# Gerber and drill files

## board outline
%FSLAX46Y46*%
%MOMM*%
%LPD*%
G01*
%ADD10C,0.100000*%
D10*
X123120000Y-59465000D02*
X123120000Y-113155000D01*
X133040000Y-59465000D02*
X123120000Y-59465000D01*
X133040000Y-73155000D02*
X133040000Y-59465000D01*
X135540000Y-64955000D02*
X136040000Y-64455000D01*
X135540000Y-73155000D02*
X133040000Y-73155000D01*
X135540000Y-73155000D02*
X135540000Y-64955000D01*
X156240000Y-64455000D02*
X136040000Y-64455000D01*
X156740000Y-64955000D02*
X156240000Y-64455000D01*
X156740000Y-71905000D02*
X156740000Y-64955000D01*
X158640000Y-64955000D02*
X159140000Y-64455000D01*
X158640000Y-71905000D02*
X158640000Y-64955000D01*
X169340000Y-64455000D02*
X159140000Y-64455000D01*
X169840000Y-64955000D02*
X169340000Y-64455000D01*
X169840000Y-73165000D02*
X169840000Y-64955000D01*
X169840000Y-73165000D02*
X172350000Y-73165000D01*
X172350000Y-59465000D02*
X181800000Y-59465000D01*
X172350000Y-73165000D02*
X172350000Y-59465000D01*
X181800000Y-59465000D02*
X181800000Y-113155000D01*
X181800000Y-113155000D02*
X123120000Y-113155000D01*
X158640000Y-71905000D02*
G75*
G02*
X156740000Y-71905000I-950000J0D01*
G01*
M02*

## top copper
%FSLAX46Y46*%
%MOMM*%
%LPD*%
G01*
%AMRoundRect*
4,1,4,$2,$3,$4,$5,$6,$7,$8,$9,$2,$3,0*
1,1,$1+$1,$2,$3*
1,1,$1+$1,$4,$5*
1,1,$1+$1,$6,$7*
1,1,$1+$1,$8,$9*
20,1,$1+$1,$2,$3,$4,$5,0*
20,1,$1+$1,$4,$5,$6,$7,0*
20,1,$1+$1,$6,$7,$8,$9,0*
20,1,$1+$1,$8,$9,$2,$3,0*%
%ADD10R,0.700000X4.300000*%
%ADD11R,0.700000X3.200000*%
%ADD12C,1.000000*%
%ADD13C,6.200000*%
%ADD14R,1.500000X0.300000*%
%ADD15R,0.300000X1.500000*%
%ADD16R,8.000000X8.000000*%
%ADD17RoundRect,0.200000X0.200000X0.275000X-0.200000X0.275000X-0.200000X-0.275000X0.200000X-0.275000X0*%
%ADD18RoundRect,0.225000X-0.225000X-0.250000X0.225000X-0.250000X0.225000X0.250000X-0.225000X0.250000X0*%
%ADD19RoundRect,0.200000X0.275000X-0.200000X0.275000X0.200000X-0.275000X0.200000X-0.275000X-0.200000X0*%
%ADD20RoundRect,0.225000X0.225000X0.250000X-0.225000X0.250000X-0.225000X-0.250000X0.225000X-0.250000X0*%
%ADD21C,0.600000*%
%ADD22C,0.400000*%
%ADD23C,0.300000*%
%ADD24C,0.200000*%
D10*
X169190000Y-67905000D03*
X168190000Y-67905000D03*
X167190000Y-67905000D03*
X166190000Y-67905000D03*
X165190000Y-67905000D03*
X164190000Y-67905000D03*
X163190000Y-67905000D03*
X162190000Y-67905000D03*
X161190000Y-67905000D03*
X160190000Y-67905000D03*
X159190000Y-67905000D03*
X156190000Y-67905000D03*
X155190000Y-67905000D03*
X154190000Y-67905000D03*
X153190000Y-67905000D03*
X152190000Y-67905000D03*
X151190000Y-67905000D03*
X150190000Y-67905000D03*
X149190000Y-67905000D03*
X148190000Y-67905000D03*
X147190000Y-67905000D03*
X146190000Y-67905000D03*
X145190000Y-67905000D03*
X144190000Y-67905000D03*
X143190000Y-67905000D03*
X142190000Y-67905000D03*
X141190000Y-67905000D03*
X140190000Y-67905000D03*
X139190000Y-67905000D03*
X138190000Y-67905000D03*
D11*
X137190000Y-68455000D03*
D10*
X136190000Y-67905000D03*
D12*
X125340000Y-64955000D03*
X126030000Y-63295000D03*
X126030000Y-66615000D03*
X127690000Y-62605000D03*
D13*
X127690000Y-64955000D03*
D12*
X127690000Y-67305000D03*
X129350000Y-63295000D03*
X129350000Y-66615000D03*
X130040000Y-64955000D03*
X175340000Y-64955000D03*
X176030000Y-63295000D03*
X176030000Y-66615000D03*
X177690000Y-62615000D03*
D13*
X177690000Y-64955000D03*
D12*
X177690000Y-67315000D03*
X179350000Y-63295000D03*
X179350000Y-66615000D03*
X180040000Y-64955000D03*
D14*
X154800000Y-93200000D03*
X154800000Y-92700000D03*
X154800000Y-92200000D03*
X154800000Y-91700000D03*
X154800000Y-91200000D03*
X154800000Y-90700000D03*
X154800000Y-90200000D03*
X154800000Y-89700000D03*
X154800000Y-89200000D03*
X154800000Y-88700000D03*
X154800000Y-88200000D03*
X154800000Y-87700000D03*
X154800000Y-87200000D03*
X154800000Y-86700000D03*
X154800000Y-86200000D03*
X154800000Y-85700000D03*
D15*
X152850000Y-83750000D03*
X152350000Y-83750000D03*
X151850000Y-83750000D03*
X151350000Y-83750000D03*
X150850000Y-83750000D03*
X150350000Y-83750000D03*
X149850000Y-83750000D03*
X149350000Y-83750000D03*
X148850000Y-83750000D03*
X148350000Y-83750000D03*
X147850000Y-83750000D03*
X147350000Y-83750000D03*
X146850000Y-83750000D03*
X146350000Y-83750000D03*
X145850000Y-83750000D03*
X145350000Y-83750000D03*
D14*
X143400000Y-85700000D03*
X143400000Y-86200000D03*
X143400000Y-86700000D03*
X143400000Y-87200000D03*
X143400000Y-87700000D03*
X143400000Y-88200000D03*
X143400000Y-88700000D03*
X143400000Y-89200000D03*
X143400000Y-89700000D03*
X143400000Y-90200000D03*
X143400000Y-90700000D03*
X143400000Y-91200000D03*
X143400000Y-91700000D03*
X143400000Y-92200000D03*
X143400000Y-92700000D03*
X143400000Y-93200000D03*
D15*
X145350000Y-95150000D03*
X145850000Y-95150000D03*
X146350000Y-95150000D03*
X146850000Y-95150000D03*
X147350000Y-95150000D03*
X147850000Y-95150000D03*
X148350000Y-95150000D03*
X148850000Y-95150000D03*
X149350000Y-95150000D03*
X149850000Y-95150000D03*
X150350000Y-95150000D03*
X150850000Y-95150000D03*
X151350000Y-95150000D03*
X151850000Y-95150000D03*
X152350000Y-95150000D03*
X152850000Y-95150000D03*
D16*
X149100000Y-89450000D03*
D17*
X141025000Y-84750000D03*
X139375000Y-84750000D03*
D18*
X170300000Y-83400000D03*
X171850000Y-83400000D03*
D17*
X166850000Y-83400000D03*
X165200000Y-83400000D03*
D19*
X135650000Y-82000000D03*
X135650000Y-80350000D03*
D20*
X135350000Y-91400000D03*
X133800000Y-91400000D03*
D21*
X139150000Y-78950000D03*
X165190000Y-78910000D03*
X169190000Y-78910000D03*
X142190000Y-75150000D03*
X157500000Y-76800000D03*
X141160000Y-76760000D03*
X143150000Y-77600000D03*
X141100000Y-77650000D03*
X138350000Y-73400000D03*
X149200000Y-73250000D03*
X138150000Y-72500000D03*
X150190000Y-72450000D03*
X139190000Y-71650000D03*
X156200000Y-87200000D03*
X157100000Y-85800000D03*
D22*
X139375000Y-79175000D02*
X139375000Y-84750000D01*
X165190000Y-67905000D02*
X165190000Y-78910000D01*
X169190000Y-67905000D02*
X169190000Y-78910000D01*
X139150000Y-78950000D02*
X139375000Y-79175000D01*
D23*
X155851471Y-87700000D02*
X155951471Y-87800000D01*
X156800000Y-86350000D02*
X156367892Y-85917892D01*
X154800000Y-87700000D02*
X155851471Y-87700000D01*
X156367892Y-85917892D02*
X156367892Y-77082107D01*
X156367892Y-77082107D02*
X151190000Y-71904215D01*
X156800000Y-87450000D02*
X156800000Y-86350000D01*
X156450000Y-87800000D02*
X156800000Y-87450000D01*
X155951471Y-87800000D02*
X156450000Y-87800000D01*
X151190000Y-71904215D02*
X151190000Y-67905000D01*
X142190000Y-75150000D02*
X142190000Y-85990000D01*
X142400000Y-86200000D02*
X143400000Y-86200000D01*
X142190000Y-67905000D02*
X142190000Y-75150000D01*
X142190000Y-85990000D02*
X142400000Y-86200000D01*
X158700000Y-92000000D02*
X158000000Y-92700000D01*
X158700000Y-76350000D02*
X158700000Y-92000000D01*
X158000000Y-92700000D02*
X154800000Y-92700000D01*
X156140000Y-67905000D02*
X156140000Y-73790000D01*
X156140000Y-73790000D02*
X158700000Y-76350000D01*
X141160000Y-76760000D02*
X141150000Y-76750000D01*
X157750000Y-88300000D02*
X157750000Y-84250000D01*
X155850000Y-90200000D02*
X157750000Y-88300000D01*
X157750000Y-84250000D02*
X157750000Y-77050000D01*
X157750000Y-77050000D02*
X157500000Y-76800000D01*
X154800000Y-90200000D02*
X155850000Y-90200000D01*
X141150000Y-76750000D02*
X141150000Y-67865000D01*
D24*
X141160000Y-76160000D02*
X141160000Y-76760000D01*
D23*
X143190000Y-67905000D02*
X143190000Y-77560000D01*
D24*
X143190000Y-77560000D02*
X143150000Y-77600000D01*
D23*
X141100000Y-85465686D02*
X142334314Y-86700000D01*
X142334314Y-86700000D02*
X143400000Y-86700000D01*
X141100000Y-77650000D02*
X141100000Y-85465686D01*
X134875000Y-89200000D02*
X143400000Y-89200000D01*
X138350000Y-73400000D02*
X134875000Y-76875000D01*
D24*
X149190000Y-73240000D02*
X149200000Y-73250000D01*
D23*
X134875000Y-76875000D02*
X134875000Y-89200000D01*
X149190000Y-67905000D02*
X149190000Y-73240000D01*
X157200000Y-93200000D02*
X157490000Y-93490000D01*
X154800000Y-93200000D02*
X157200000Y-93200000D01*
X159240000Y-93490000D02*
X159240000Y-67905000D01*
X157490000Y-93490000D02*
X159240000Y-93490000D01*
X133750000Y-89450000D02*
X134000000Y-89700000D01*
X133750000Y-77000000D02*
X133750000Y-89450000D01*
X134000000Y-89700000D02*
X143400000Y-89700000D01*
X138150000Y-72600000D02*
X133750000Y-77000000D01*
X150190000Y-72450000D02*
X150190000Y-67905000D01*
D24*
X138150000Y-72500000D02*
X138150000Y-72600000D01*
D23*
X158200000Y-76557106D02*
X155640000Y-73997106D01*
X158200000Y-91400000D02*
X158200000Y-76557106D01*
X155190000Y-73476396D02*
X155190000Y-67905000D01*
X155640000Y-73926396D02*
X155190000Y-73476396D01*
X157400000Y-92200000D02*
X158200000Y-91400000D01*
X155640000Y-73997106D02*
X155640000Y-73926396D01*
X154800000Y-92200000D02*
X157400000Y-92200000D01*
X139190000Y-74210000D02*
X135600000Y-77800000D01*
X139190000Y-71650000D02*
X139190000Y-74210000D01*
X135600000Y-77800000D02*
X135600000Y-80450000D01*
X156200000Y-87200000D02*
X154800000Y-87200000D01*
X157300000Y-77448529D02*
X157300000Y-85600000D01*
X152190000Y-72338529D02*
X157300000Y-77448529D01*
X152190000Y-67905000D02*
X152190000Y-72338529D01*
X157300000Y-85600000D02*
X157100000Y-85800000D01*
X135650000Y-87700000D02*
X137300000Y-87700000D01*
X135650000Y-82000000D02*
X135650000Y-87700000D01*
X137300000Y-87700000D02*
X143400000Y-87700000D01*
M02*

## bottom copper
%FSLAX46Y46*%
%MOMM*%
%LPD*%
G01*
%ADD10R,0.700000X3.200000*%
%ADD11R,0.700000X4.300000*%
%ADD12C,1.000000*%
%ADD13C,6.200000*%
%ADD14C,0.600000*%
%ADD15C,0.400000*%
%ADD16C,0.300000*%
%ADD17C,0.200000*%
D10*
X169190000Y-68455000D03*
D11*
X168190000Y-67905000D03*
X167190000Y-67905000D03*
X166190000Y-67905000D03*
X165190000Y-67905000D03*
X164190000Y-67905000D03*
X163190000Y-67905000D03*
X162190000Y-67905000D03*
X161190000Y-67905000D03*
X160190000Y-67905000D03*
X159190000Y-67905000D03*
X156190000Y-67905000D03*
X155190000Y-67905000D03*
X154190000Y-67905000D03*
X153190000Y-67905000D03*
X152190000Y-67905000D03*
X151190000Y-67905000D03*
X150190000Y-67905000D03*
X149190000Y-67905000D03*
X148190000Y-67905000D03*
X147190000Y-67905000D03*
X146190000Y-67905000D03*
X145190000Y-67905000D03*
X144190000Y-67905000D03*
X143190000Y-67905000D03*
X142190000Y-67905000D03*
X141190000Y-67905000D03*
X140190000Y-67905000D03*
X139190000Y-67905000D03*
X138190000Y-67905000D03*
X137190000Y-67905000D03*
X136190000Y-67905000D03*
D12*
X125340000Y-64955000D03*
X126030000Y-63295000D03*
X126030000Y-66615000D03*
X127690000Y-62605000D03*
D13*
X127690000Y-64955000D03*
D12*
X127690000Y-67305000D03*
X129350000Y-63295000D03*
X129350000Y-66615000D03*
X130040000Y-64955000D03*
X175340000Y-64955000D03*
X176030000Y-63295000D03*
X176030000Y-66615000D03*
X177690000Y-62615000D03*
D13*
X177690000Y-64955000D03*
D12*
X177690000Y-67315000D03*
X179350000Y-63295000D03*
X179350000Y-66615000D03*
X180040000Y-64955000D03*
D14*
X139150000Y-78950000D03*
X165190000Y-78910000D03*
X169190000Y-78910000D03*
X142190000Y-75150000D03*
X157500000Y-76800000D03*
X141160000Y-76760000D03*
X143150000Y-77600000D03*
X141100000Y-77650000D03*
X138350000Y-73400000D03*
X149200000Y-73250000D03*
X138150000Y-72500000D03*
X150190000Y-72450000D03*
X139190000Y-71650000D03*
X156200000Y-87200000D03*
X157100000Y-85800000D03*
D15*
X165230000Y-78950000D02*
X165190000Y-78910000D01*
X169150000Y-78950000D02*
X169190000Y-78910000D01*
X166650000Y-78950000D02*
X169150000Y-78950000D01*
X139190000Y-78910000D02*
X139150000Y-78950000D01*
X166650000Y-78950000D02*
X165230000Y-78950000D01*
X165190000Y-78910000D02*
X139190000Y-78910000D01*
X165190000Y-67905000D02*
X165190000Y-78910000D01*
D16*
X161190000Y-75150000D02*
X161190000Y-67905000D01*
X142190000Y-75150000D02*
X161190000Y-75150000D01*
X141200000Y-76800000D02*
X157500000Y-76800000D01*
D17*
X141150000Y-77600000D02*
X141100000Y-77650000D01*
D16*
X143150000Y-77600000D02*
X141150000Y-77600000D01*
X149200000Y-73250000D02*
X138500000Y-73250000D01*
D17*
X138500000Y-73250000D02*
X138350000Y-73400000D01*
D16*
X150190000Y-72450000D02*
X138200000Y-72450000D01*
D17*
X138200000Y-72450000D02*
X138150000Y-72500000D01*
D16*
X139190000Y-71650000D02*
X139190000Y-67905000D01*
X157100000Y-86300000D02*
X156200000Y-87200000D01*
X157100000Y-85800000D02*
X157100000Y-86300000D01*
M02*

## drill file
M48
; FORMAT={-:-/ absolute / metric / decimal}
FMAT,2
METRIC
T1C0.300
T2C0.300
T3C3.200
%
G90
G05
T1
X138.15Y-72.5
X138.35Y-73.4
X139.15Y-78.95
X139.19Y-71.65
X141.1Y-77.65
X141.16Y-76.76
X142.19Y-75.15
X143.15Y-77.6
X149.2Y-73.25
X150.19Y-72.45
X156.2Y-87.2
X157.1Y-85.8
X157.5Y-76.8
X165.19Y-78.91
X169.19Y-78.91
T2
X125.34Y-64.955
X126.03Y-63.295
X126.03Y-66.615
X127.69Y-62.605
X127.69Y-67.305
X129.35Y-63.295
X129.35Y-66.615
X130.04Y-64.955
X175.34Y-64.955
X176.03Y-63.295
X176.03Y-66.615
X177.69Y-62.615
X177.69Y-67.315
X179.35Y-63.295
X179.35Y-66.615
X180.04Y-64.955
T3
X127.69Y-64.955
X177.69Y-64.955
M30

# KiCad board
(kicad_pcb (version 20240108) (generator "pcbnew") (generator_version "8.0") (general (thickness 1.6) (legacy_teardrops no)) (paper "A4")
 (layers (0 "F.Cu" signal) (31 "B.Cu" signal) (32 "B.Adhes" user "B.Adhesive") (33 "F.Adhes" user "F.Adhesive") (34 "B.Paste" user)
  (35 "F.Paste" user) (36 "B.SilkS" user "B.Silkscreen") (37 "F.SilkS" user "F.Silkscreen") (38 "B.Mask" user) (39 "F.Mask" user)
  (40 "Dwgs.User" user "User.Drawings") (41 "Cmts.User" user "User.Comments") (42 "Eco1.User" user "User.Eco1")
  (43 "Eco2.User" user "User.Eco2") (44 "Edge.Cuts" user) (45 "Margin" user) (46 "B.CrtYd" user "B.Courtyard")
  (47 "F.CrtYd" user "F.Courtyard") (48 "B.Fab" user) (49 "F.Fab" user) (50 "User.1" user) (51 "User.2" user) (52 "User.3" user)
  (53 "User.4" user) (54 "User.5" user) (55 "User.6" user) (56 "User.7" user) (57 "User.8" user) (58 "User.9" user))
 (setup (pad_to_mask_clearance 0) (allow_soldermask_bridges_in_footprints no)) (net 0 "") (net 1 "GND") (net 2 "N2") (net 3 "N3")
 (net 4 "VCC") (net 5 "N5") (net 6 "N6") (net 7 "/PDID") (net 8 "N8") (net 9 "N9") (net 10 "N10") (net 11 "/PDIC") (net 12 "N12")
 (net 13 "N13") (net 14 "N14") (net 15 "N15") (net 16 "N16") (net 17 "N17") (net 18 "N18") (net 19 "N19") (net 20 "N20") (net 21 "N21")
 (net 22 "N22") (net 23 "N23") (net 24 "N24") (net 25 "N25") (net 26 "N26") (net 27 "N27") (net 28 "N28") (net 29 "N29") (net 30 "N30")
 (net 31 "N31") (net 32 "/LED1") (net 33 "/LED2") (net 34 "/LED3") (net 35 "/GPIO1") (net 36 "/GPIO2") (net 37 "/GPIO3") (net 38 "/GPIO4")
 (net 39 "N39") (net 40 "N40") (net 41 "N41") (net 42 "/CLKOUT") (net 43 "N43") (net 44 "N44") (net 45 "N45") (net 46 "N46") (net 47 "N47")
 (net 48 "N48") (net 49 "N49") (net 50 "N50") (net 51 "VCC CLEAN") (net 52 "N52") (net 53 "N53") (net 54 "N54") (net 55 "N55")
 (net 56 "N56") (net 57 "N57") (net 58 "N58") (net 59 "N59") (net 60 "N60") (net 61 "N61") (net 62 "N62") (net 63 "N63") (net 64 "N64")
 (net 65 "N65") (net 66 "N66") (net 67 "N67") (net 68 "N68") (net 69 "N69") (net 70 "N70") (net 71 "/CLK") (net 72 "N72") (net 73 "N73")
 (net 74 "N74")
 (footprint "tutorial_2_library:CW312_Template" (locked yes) (layer "F.Cu") (at 127.69 64.955)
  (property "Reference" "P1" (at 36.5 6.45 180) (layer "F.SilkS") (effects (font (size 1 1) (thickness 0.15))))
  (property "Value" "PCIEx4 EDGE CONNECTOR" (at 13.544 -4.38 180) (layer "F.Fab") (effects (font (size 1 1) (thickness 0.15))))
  (fp_line (start -4.57 -5.49) (end -4.57 48.2) (stroke (width 0.1) (type default)) (layer "Edge.Cuts"))
  (fp_line (start 5.35 -5.49) (end -4.57 -5.49) (stroke (width 0.1) (type default)) (layer "Edge.Cuts"))
  (fp_line (start 5.35 8.2) (end 5.35 -5.49) (stroke (width 0.1) (type default)) (layer "Edge.Cuts"))
  (fp_line (start 7.85 0) (end 8.35 -0.5) (stroke (width 0.1) (type solid)) (layer "Edge.Cuts"))
  (fp_line (start 7.85 8.2) (end 5.35 8.2) (stroke (width 0.1) (type default)) (layer "Edge.Cuts"))
  (fp_line (start 7.85 8.2) (end 7.85 0) (stroke (width 0.1) (type solid)) (layer "Edge.Cuts"))
  (fp_line (start 28.55 -0.5) (end 8.35 -0.5) (stroke (width 0.1) (type solid)) (layer "Edge.Cuts"))
  (fp_line (start 29.05 0) (end 28.55 -0.5) (stroke (width 0.1) (type solid)) (layer "Edge.Cuts"))
  (fp_line (start 29.05 6.95) (end 29.05 0) (stroke (width 0.1) (type solid)) (layer "Edge.Cuts"))
  (fp_line (start 30.95 0) (end 31.45 -0.5) (stroke (width 0.1) (type solid)) (layer "Edge.Cuts"))
  (fp_line (start 30.95 6.95) (end 30.95 0) (stroke (width 0.1) (type solid)) (layer "Edge.Cuts"))
  (fp_line (start 41.65 -0.5) (end 31.45 -0.5) (stroke (width 0.1) (type solid)) (layer "Edge.Cuts"))
  (fp_line (start 42.15 0) (end 41.65 -0.5) (stroke (width 0.1) (type solid)) (layer "Edge.Cuts"))
  (fp_line (start 42.15 8.21) (end 42.15 0) (stroke (width 0.1) (type solid)) (layer "Edge.Cuts"))
  (fp_line (start 42.15 8.21) (end 44.66 8.21) (stroke (width 0.1) (type default)) (layer "Edge.Cuts"))
  (fp_line (start 44.66 -5.49) (end 54.11 -5.49) (stroke (width 0.1) (type default)) (layer "Edge.Cuts"))
  (fp_line (start 44.66 8.21) (end 44.66 -5.49) (stroke (width 0.1) (type default)) (layer "Edge.Cuts"))
  (fp_line (start 54.11 -5.49) (end 54.11 48.2) (stroke (width 0.1) (type default)) (layer "Edge.Cuts"))
  (fp_line (start 54.11 48.2) (end -4.57 48.2) (stroke (width 0.1) (type default)) (layer "Edge.Cuts"))
  (fp_arc (start 30.95 6.95) (mid 30 7.9) (end 29.05 6.95) (stroke (width 0.1) (type solid)) (layer "Edge.Cuts"))
  (pad "A1" connect rect (at 41.5 3.5 180) (size 0.7 3.2) (layers "B.Cu" "B.Mask") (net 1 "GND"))
  (pad "A2" connect rect (at 40.5 2.95 180) (size 0.7 4.3) (layers "B.Cu" "B.Mask") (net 1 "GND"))
  (pad "A3" connect rect (at 39.5 2.95 180) (size 0.7 4.3) (layers "B.Cu" "B.Mask") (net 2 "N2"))
  (pad "A4" connect rect (at 38.5 2.95 180) (size 0.7 4.3) (layers "B.Cu" "B.Mask") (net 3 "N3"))
  (pad "A5" connect rect (at 37.5 2.95 180) (size 0.7 4.3) (layers "B.Cu" "B.Mask") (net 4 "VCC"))
  (pad "A6" connect rect (at 36.5 2.95 180) (size 0.7 4.3) (layers "B.Cu" "B.Mask") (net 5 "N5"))
  (pad "A7" connect rect (at 35.5 2.95 180) (size 0.7 4.3) (layers "B.Cu" "B.Mask") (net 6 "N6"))
  (pad "A8" connect rect (at 34.5 2.95 180) (size 0.7 4.3) (layers "B.Cu" "B.Mask") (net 1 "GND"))
  (pad "A9" connect rect (at 33.5 2.95 180) (size 0.7 4.3) (layers "B.Cu" "B.Mask") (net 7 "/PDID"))
  (pad "A10" connect rect (at 32.5 2.95 180) (size 0.7 4.3) (layers "B.Cu" "B.Mask") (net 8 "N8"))
  (pad "A11" connect rect (at 31.5 2.95 180) (size 0.7 4.3) (layers "B.Cu" "B.Mask") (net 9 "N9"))
  (pad "A12" connect rect (at 28.5 2.95 180) (size 0.7 4.3) (layers "B.Cu" "B.Mask") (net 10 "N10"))
  (pad "A13" connect rect (at 27.5 2.95 180) (size 0.7 4.3) (layers "B.Cu" "B.Mask") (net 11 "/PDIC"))
  (pad "A14" connect rect (at 26.5 2.95 180) (size 0.7 4.3) (layers "B.Cu" "B.Mask") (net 1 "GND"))
  (pad "A15" connect rect (at 25.5 2.95 180) (size 0.7 4.3) (layers "B.Cu" "B.Mask") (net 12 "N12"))
  (pad "A16" connect rect (at 24.5 2.95 180) (size 0.7 4.3) (layers "B.Cu" "B.Mask") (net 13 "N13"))
  (pad "A17" connect rect (at 23.5 2.95 180) (size 0.7 4.3) (layers "B.Cu" "B.Mask") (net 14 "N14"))
  (pad "A18" connect rect (at 22.5 2.95 180) (size 0.7 4.3) (layers "B.Cu" "B.Mask") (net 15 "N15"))
  (pad "A19" connect rect (at 21.5 2.95 180) (size 0.7 4.3) (layers "B.Cu" "B.Mask") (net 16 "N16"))
  (pad "A20" connect rect (at 20.5 2.95 180) (size 0.7 4.3) (layers "B.Cu" "B.Mask") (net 1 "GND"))
  (pad "A21" connect rect (at 19.5 2.95 180) (size 0.7 4.3) (layers "B.Cu" "B.Mask") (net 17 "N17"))
  (pad "A22" connect rect (at 18.5 2.95 180) (size 0.7 4.3) (layers "B.Cu" "B.Mask") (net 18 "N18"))
  (pad "A23" connect rect (at 17.5 2.95 180) (size 0.7 4.3) (layers "B.Cu" "B.Mask") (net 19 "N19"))
  (pad "A24" connect rect (at 16.5 2.95 180) (size 0.7 4.3) (layers "B.Cu" "B.Mask") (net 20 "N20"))
  (pad "A25" connect rect (at 15.5 2.95 180) (size 0.7 4.3) (layers "B.Cu" "B.Mask") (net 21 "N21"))
  (pad "A26" connect rect (at 14.5 2.95 180) (size 0.7 4.3) (layers "B.Cu" "B.Mask") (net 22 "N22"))
  (pad "A27" connect rect (at 13.5 2.95 180) (size 0.7 4.3) (layers "B.Cu" "B.Mask") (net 1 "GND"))
  (pad "A28" connect rect (at 12.5 2.95 180) (size 0.7 4.3) (layers "B.Cu" "B.Mask") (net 1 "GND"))
  (pad "A29" connect rect (at 11.5 2.95 180) (size 0.7 4.3) (layers "B.Cu" "B.Mask") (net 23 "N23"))
  (pad "A30" connect rect (at 10.5 2.95 180) (size 0.7 4.3) (layers "B.Cu" "B.Mask") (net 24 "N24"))
  (pad "A31" connect rect (at 9.5 2.95 180) (size 0.7 4.3) (layers "B.Cu" "B.Mask") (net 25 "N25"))
  (pad "A32" connect rect (at 8.5 2.95 180) (size 0.7 4.3) (layers "B.Cu" "B.Mask") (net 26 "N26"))
  (pad "B1" connect rect (at 41.5 2.95 180) (size 0.7 4.3) (layers "F.Cu" "F.Mask") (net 4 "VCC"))
  (pad "B2" connect rect (at 40.5 2.95 180) (size 0.7 4.3) (layers "F.Cu" "F.Mask") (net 2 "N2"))
  (pad "B3" connect rect (at 39.5 2.95 180) (size 0.7 4.3) (layers "F.Cu" "F.Mask") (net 1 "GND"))
  (pad "B4" connect rect (at 38.5 2.95 180) (size 0.7 4.3) (layers "F.Cu" "F.Mask") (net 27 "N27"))
  (pad "B5" connect rect (at 37.5 2.95 180) (size 0.7 4.3) (layers "F.Cu" "F.Mask") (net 4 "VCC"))
  (pad "B6" connect rect (at 36.5 2.95 180) (size 0.7 4.3) (layers "F.Cu" "F.Mask") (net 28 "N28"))
  (pad "B7" connect rect (at 35.5 2.95 180) (size 0.7 4.3) (layers "F.Cu" "F.Mask") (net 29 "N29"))
  (pad "B8" connect rect (at 34.5 2.95 180) (size 0.7 4.3) (layers "F.Cu" "F.Mask") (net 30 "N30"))
  (pad "B9" connect rect (at 33.5 2.95 180) (size 0.7 4.3) (layers "F.Cu" "F.Mask") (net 1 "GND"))
  (pad "B10" connect rect (at 32.5 2.95 180) (size 0.7 4.3) (layers "F.Cu" "F.Mask") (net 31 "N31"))
  (pad "B11" connect rect (at 31.5 2.95 180) (size 0.7 4.3) (layers "F.Cu" "F.Mask") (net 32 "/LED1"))
  (pad "B12" connect rect (at 28.5 2.95 180) (size 0.7 4.3) (layers "F.Cu" "F.Mask") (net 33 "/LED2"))
  (pad "B13" connect rect (at 27.5 2.95 180) (size 0.7 4.3) (layers "F.Cu" "F.Mask") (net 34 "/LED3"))
  (pad "B14" connect rect (at 26.5 2.95 180) (size 0.7 4.3) (layers "F.Cu" "F.Mask") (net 11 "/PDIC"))
  (pad "B15" connect rect (at 25.5 2.95 180) (size 0.7 4.3) (layers "F.Cu" "F.Mask") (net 1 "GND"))
  (pad "B16" connect rect (at 24.5 2.95 180) (size 0.7 4.3) (layers "F.Cu" "F.Mask") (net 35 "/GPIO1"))
  (pad "B17" connect rect (at 23.5 2.95 180) (size 0.7 4.3) (layers "F.Cu" "F.Mask") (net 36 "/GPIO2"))
  (pad "B18" connect rect (at 22.5 2.95 180) (size 0.7 4.3) (layers "F.Cu" "F.Mask") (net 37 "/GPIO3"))
  (pad "B19" connect rect (at 21.5 2.95 180) (size 0.7 4.3) (layers "F.Cu" "F.Mask") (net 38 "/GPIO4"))
  (pad "B20" connect rect (at 20.5 2.95 180) (size 0.7 4.3) (layers "F.Cu" "F.Mask") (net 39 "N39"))
  (pad "B21" connect rect (at 19.5 2.95 180) (size 0.7 4.3) (layers "F.Cu" "F.Mask") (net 1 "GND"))
  (pad "B22" connect rect (at 18.5 2.95 180) (size 0.7 4.3) (layers "F.Cu" "F.Mask") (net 1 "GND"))
  (pad "B23" connect rect (at 17.5 2.95 180) (size 0.7 4.3) (layers "F.Cu" "F.Mask") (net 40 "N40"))
  (pad "B24" connect rect (at 16.5 2.95 180) (size 0.7 4.3) (layers "F.Cu" "F.Mask") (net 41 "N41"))
  (pad "B25" connect rect (at 15.5 2.95 180) (size 0.7 4.3) (layers "F.Cu" "F.Mask") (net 11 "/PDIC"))
  (pad "B26" connect rect (at 14.5 2.95 180) (size 0.7 4.3) (layers "F.Cu" "F.Mask") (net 7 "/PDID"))
  (pad "B27" connect rect (at 13.5 2.95 180) (size 0.7 4.3) (layers "F.Cu" "F.Mask") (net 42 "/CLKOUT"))
  (pad "B28" connect rect (at 12.5 2.95 180) (size 0.7 4.3) (layers "F.Cu" "F.Mask") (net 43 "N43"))
  (pad "B29" connect rect (at 11.5 2.95 180) (size 0.7 4.3) (layers "F.Cu" "F.Mask") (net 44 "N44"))
  (pad "B30" connect rect (at 10.5 2.95 180) (size 0.7 4.3) (layers "F.Cu" "F.Mask") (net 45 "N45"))
  (pad "B31" connect rect (at 9.5 3.5 180) (size 0.7 3.2) (layers "F.Cu" "F.Mask") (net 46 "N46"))
  (pad "B32" connect rect (at 8.5 2.95 180) (size 0.7 4.3) (layers "F.Cu" "F.Mask") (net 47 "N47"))
  (pad "MH" thru_hole circle (at -2.35 0) (size 1 1) (drill 0.3) (layers "*.Cu" "*.Mask") (remove_unused_layers no))
  (pad "MH" thru_hole circle (at -1.66 -1.66) (size 1 1) (drill 0.3) (layers "*.Cu" "*.Mask") (remove_unused_layers no))
  (pad "MH" thru_hole circle (at -1.66 1.66) (size 1 1) (drill 0.3) (layers "*.Cu" "*.Mask") (remove_unused_layers no))
  (pad "MH" thru_hole circle (at 0 -2.35) (size 1 1) (drill 0.3) (layers "*.Cu" "*.Mask") (remove_unused_layers no))
  (pad "MH" thru_hole circle (at 0 0) (size 6.2 6.2) (drill 3.2) (layers "*.Cu" "*.Mask") (remove_unused_layers no))
  (pad "MH" thru_hole circle (at 0 2.35) (size 1 1) (drill 0.3) (layers "*.Cu" "*.Mask") (remove_unused_layers no))
  (pad "MH" thru_hole circle (at 1.66 -1.66) (size 1 1) (drill 0.3) (layers "*.Cu" "*.Mask") (remove_unused_layers no))
  (pad "MH" thru_hole circle (at 1.66 1.66) (size 1 1) (drill 0.3) (layers "*.Cu" "*.Mask") (remove_unused_layers no))
  (pad "MH" thru_hole circle (at 2.35 0) (size 1 1) (drill 0.3) (layers "*.Cu" "*.Mask") (remove_unused_layers no))
  (pad "MH" thru_hole circle (at 47.65 0) (size 1 1) (drill 0.3) (layers "*.Cu" "*.Mask") (remove_unused_layers no))
  (pad "MH" thru_hole circle (at 48.34 -1.66) (size 1 1) (drill 0.3) (layers "*.Cu" "*.Mask") (remove_unused_layers no))
  (pad "MH" thru_hole circle (at 48.34 1.66) (size 1 1) (drill 0.3) (layers "*.Cu" "*.Mask") (remove_unused_layers no))
  (pad "MH" thru_hole circle (at 50 -2.34) (size 1 1) (drill 0.3) (layers "*.Cu" "*.Mask") (remove_unused_layers no))
  (pad "MH" thru_hole circle (at 50 0) (size 6.2 6.2) (drill 3.2) (layers "*.Cu" "*.Mask") (remove_unused_layers no))
  (pad "MH" thru_hole circle (at 50 2.36) (size 1 1) (drill 0.3) (layers "*.Cu" "*.Mask") (remove_unused_layers no))
  (pad "MH" thru_hole circle (at 51.66 -1.66) (size 1 1) (drill 0.3) (layers "*.Cu" "*.Mask") (remove_unused_layers no))
  (pad "MH" thru_hole circle (at 51.66 1.66) (size 1 1) (drill 0.3) (layers "*.Cu" "*.Mask") (remove_unused_layers no))
  (pad "MH" thru_hole circle (at 52.35 0) (size 1 1) (drill 0.3) (layers "*.Cu" "*.Mask") (remove_unused_layers no)))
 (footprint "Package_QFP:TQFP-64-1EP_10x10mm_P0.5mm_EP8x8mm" (layer "F.Cu") (at 149.1 89.45 180)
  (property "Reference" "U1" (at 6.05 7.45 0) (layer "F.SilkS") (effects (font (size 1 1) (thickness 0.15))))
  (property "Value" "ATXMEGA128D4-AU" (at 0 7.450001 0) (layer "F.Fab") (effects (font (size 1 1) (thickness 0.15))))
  (pad "" smd rect (at -3.2 -3.2 180) (size 1.24 1.24) (layers "F.Paste"))
  (pad "" smd rect (at -3.2 -1.6 180) (size 1.24 1.24) (layers "F.Paste"))
  (pad "" smd rect (at -3.2 0 180) (size 1.24 1.24) (layers "F.Paste"))
  (pad "" smd rect (at -3.2 1.6 180) (size 1.24 1.24) (layers "F.Paste"))
  (pad "" smd rect (at -3.2 3.2 180) (size 1.24 1.24) (layers "F.Paste"))
  (pad "" smd rect (at -1.6 -3.2 180) (size 1.24 1.24) (layers "F.Paste"))
  (pad "" smd rect (at -1.6 -1.6 180) (size 1.24 1.24) (layers "F.Paste"))
  (pad "" smd rect (at -1.6 0 180) (size 1.24 1.24) (layers "F.Paste"))
  (pad "" smd rect (at -1.6 1.6 180) (size 1.24 1.24) (layers "F.Paste"))
  (pad "" smd rect (at -1.6 3.2 180) (size 1.24 1.24) (layers "F.Paste"))
  (pad "" smd rect (at 0 -3.2 180) (size 1.24 1.24) (layers "F.Paste"))
  (pad "" smd rect (at 0 -1.6 180) (size 1.24 1.24) (layers "F.Paste"))
  (pad "" smd rect (at 0 0 180) (size 1.24 1.24) (layers "F.Paste"))
  (pad "" smd rect (at 0 1.6 180) (size 1.24 1.24) (layers "F.Paste"))
  (pad "" smd rect (at 0 3.2 180) (size 1.24 1.24) (layers "F.Paste"))
  (pad "" smd rect (at 1.6 -3.2 180) (size 1.24 1.24) (layers "F.Paste"))
  (pad "" smd rect (at 1.6 -1.6 180) (size 1.24 1.24) (layers "F.Paste"))
  (pad "" smd rect (at 1.6 0 180) (size 1.24 1.24) (layers "F.Paste"))
  (pad "" smd rect (at 1.6 1.6 180) (size 1.24 1.24) (layers "F.Paste"))
  (pad "" smd rect (at 1.6 3.2 180) (size 1.24 1.24) (layers "F.Paste"))
  (pad "" smd rect (at 3.2 -3.2 180) (size 1.24 1.24) (layers "F.Paste"))
  (pad "" smd rect (at 3.2 -1.6 180) (size 1.24 1.24) (layers "F.Paste"))
  (pad "" smd rect (at 3.2 0 180) (size 1.24 1.24) (layers "F.Paste"))
  (pad "" smd rect (at 3.2 1.6 180) (size 1.24 1.24) (layers "F.Paste"))
  (pad "" smd rect (at 3.2 3.2 180) (size 1.24 1.24) (layers "F.Paste"))
  (pad "1" smd rect (at -5.7 -3.75 180) (size 1.5 0.3) (layers "F.Cu" "F.Paste" "F.Mask") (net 32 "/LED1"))
  (pad "2" smd rect (at -5.7 -3.25 180) (size 1.5 0.3) (layers "F.Cu" "F.Paste" "F.Mask") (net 33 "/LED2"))
  (pad "3" smd rect (at -5.7 -2.75 180) (size 1.5 0.3) (layers "F.Cu" "F.Paste" "F.Mask") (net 34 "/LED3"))
  (pad "4" smd rect (at -5.7 -2.25 180) (size 1.5 0.3) (layers "F.Cu" "F.Paste" "F.Mask") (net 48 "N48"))
  (pad "5" smd rect (at -5.7 -1.75 180) (size 1.5 0.3) (layers "F.Cu" "F.Paste" "F.Mask") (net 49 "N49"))
  (pad "6" smd rect (at -5.7 -1.25 180) (size 1.5 0.3) (layers "F.Cu" "F.Paste" "F.Mask") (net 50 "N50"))
  (pad "7" smd rect (at -5.7 -0.75 180) (size 1.5 0.3) (layers "F.Cu" "F.Paste" "F.Mask") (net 42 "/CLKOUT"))
  (pad "8" smd rect (at -5.7 -0.25 180) (size 1.5 0.3) (layers "F.Cu" "F.Paste" "F.Mask") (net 1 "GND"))
  (pad "9" smd rect (at -5.7 0.25 180) (size 1.5 0.3) (layers "F.Cu" "F.Paste" "F.Mask") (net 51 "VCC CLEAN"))
  (pad "10" smd rect (at -5.7 0.75 180) (size 1.5 0.3) (layers "F.Cu" "F.Paste" "F.Mask") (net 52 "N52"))
  (pad "11" smd rect (at -5.7 1.25 180) (size 1.5 0.3) (layers "F.Cu" "F.Paste" "F.Mask") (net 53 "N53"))
  (pad "12" smd rect (at -5.7 1.75 180) (size 1.5 0.3) (layers "F.Cu" "F.Paste" "F.Mask") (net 36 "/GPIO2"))
  (pad "13" smd rect (at -5.7 2.25 180) (size 1.5 0.3) (layers "F.Cu" "F.Paste" "F.Mask") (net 35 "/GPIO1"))
  (pad "14" smd rect (at -5.7 2.75 180) (size 1.5 0.3) (layers "F.Cu" "F.Paste" "F.Mask") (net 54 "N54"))
  (pad "15" smd rect (at -5.7 3.25 180) (size 1.5 0.3) (layers "F.Cu" "F.Paste" "F.Mask") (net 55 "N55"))
  (pad "16" smd rect (at -5.7 3.75 180) (size 1.5 0.3) (layers "F.Cu" "F.Paste" "F.Mask") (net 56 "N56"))
  (pad "17" smd rect (at -3.75 5.7 270) (size 1.5 0.3) (layers "F.Cu" "F.Paste" "F.Mask") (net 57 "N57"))
  (pad "18" smd rect (at -3.25 5.7 270) (size 1.5 0.3) (layers "F.Cu" "F.Paste" "F.Mask") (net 1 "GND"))
  (pad "19" smd rect (at -2.75 5.7 270) (size 1.5 0.3) (layers "F.Cu" "F.Paste" "F.Mask") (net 51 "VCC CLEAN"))
  (pad "20" smd rect (at -2.25 5.7 270) (size 1.5 0.3) (layers "F.Cu" "F.Paste" "F.Mask") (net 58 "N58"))
  (pad "21" smd rect (at -1.75 5.7 270) (size 1.5 0.3) (layers "F.Cu" "F.Paste" "F.Mask") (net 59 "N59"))
  (pad "22" smd rect (at -1.25 5.7 270) (size 1.5 0.3) (layers "F.Cu" "F.Paste" "F.Mask") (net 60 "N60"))
  (pad "23" smd rect (at -0.75 5.7 270) (size 1.5 0.3) (layers "F.Cu" "F.Paste" "F.Mask") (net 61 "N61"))
  (pad "24" smd rect (at -0.25 5.7 270) (size 1.5 0.3) (layers "F.Cu" "F.Paste" "F.Mask") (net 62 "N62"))
  (pad "25" smd rect (at 0.25 5.7 270) (size 1.5 0.3) (layers "F.Cu" "F.Paste" "F.Mask") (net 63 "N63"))
  (pad "26" smd rect (at 0.75 5.7 270) (size 1.5 0.3) (layers "F.Cu" "F.Paste" "F.Mask") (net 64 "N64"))
  (pad "27" smd rect (at 1.25 5.7 270) (size 1.5 0.3) (layers "F.Cu" "F.Paste" "F.Mask") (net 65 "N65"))
  (pad "28" smd rect (at 1.75 5.7 270) (size 1.5 0.3) (layers "F.Cu" "F.Paste" "F.Mask") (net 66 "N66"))
  (pad "29" smd rect (at 2.25 5.7 270) (size 1.5 0.3) (layers "F.Cu" "F.Paste" "F.Mask") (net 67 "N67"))
  (pad "30" smd rect (at 2.75 5.7 270) (size 1.5 0.3) (layers "F.Cu" "F.Paste" "F.Mask") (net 1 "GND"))
  (pad "31" smd rect (at 3.25 5.7 270) (size 1.5 0.3) (layers "F.Cu" "F.Paste" "F.Mask") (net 51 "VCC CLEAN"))
  (pad "32" smd rect (at 3.75 5.7 270) (size 1.5 0.3) (layers "F.Cu" "F.Paste" "F.Mask") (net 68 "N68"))
  (pad "33" smd rect (at 5.7 3.75 180) (size 1.5 0.3) (layers "F.Cu" "F.Paste" "F.Mask") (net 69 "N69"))
  (pad "34" smd rect (at 5.7 3.25 180) (size 1.5 0.3) (layers "F.Cu" "F.Paste" "F.Mask") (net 7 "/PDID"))
  (pad "35" smd rect (at 5.7 2.75 180) (size 1.5 0.3) (layers "F.Cu" "F.Paste" "F.Mask") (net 11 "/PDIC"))
  (pad "36" smd rect (at 5.7 2.25 180) (size 1.5 0.3) (layers "F.Cu" "F.Paste" "F.Mask") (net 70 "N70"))
  (pad "37" smd rect (at 5.7 1.75 180) (size 1.5 0.3) (layers "F.Cu" "F.Paste" "F.Mask") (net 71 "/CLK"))
  (pad "38" smd rect (at 5.7 1.25 180) (size 1.5 0.3) (layers "F.Cu" "F.Paste" "F.Mask") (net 1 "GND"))
  (pad "39" smd rect (at 5.7 0.75 180) (size 1.5 0.3) (layers "F.Cu" "F.Paste" "F.Mask") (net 4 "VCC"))
  (pad "40" smd rect (at 5.7 0.25 180) (size 1.5 0.3) (layers "F.Cu" "F.Paste" "F.Mask") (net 38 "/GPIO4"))
  (pad "41" smd rect (at 5.7 -0.25 180) (size 1.5 0.3) (layers "F.Cu" "F.Paste" "F.Mask") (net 37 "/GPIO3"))
  (pad "42" smd rect (at 5.7 -0.75 180) (size 1.5 0.3) (layers "F.Cu" "F.Paste" "F.Mask") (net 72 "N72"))
  (pad "43" smd rect (at 5.7 -1.25 180) (size 1.5 0.3) (layers "F.Cu" "F.Paste" "F.Mask") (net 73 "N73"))
  (pad "44" smd rect (at 5.7 -1.75 180) (size 1.5 0.3) (layers "F.Cu" "F.Paste" "F.Mask") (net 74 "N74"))
  (pad "45" smd rect (at 5.7 -2.25 180) (size 1.5 0.3) (layers "F.Cu" "F.Paste" "F.Mask"))
  (pad "46" smd rect (at 5.7 -2.75 180) (size 1.5 0.3) (layers "F.Cu" "F.Paste" "F.Mask"))
  (pad "47" smd rect (at 5.7 -3.25 180) (size 1.5 0.3) (layers "F.Cu" "F.Paste" "F.Mask"))
  (pad "48" smd rect (at 5.7 -3.75 180) (size 1.5 0.3) (layers "F.Cu" "F.Paste" "F.Mask"))
  (pad "49" smd rect (at 3.75 -5.7 270) (size 1.5 0.3) (layers "F.Cu" "F.Paste" "F.Mask"))
  (pad "50" smd rect (at 3.25 -5.7 270) (size 1.5 0.3) (layers "F.Cu" "F.Paste" "F.Mask"))
  (pad "51" smd rect (at 2.75 -5.7 270) (size 1.5 0.3) (layers "F.Cu" "F.Paste" "F.Mask"))
  (pad "52" smd rect (at 2.25 -5.7 270) (size 1.5 0.3) (layers "F.Cu" "F.Paste" "F.Mask"))
  (pad "53" smd rect (at 1.75 -5.7 270) (size 1.5 0.3) (layers "F.Cu" "F.Paste" "F.Mask"))
  (pad "54" smd rect (at 1.25 -5.7 270) (size 1.5 0.3) (layers "F.Cu" "F.Paste" "F.Mask"))
  (pad "55" smd rect (at 0.75 -5.7 270) (size 1.5 0.3) (layers "F.Cu" "F.Paste" "F.Mask"))
  (pad "56" smd rect (at 0.25 -5.7 270) (size 1.5 0.3) (layers "F.Cu" "F.Paste" "F.Mask"))
  (pad "57" smd rect (at -0.25 -5.7 270) (size 1.5 0.3) (layers "F.Cu" "F.Paste" "F.Mask"))
  (pad "58" smd rect (at -0.75 -5.7 270) (size 1.5 0.3) (layers "F.Cu" "F.Paste" "F.Mask"))
  (pad "59" smd rect (at -1.25 -5.7 270) (size 1.5 0.3) (layers "F.Cu" "F.Paste" "F.Mask"))
  (pad "60" smd rect (at -1.75 -5.7 270) (size 1.5 0.3) (layers "F.Cu" "F.Paste" "F.Mask"))
  (pad "61" smd rect (at -2.25 -5.7 270) (size 1.5 0.3) (layers "F.Cu" "F.Paste" "F.Mask"))
  (pad "62" smd rect (at -2.75 -5.7 270) (size 1.5 0.3) (layers "F.Cu" "F.Paste" "F.Mask"))
  (pad "63" smd rect (at -3.25 -5.7 270) (size 1.5 0.3) (layers "F.Cu" "F.Paste" "F.Mask"))
  (pad "64" smd rect (at -3.75 -5.7 270) (size 1.5 0.3) (layers "F.Cu" "F.Paste" "F.Mask"))
  (pad "65" smd rect (at 0 0 180) (size 8 8) (layers "F.Cu" "F.Mask")))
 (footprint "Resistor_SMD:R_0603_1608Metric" (layer "F.Cu") (at 140.2 84.75 180)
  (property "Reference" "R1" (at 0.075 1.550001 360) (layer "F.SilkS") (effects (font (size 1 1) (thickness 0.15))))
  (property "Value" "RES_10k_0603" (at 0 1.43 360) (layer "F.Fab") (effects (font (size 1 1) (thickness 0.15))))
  (pad "1" smd roundrect (at -0.825 0 180) (size 0.8 0.95) (layers "F.Cu" "F.Paste" "F.Mask") (roundrect_rratio 0.25) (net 11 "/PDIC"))
  (pad "2" smd roundrect (at 0.825 0 180) (size 0.8 0.95) (layers "F.Cu" "F.Paste" "F.Mask") (roundrect_rratio 0.25) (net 4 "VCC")))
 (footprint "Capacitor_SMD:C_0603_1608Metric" (layer "F.Cu") (at 171.075 83.4)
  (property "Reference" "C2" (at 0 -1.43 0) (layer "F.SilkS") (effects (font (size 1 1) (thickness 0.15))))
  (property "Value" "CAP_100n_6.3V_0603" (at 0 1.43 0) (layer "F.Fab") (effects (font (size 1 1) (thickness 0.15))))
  (pad "1" smd roundrect (at -0.775 0) (size 0.9 0.95) (layers "F.Cu" "F.Paste" "F.Mask") (roundrect_rratio 0.25) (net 2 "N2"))
  (pad "2" smd roundrect (at 0.775 0) (size 0.9 0.95) (layers "F.Cu" "F.Paste" "F.Mask") (roundrect_rratio 0.25) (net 1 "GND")))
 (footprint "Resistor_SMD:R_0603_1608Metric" (layer "F.Cu") (at 166.025 83.4 180)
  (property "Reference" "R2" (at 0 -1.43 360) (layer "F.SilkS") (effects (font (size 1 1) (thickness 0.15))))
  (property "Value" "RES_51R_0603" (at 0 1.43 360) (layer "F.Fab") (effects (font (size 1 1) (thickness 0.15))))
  (pad "1" smd roundrect (at -0.825 0 180) (size 0.8 0.95) (layers "F.Cu" "F.Paste" "F.Mask") (roundrect_rratio 0.25) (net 2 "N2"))
  (pad "2" smd roundrect (at 0.825 0 180) (size 0.8 0.95) (layers "F.Cu" "F.Paste" "F.Mask") (roundrect_rratio 0.25) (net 4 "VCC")))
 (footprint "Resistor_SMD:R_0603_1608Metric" (layer "F.Cu") (at 135.65 81.175 90)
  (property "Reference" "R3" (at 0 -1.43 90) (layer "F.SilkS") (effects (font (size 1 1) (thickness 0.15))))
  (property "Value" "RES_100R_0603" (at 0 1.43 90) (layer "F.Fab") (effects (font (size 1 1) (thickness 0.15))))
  (pad "1" smd roundrect (at -0.825 0 90) (size 0.8 0.95) (layers "F.Cu" "F.Paste" "F.Mask") (roundrect_rratio 0.25) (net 71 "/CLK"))
  (pad "2" smd roundrect (at 0.825 0 90) (size 0.8 0.95) (layers "F.Cu" "F.Paste" "F.Mask") (roundrect_rratio 0.25) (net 23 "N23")))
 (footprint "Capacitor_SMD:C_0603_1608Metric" (layer "F.Cu") (at 134.575 91.4 180)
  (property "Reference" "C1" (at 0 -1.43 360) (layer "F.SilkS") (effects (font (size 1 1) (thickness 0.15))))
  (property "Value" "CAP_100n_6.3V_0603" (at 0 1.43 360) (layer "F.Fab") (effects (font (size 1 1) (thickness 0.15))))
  (pad "1" smd roundrect (at -0.775 0 180) (size 0.9 0.95) (layers "F.Cu" "F.Paste" "F.Mask") (roundrect_rratio 0.25) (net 1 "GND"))
  (pad "2" smd roundrect (at 0.775 0 180) (size 0.9 0.95) (layers "F.Cu" "F.Paste" "F.Mask") (roundrect_rratio 0.25) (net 4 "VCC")))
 (segment (start 139.375 79.175) (end 139.375 84.75) (width 0.4) (layer "F.Cu") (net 4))
 (segment (start 165.19 67.905) (end 165.19 78.91) (width 0.4) (layer "F.Cu") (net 4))
 (segment (start 169.19 67.905) (end 169.19 78.91) (width 0.4) (layer "F.Cu") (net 4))
 (segment (start 139.15 78.95) (end 139.375 79.175) (width 0.4) (layer "F.Cu") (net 4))
 (via (at 139.15 78.95) (size 0.6) (drill 0.3) (layers "F.Cu" "B.Cu") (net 4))
 (via (at 165.19 78.91) (size 0.6) (drill 0.3) (layers "F.Cu" "B.Cu") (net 4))
 (via (at 169.19 78.91) (size 0.6) (drill 0.3) (layers "F.Cu" "B.Cu") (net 4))
 (segment (start 165.23 78.95) (end 165.19 78.91) (width 0.4) (layer "B.Cu") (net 4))
 (segment (start 169.15 78.95) (end 169.19 78.91) (width 0.4) (layer "B.Cu") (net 4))
 (segment (start 166.65 78.95) (end 169.15 78.95) (width 0.4) (layer "B.Cu") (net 4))
 (segment (start 139.19 78.91) (end 139.15 78.95) (width 0.4) (layer "B.Cu") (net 4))
 (segment (start 166.65 78.95) (end 165.23 78.95) (width 0.4) (layer "B.Cu") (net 4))
 (segment (start 165.19 78.91) (end 139.19 78.91) (width 0.4) (layer "B.Cu") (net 4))
 (segment (start 165.19 67.905) (end 165.19 78.91) (width 0.4) (layer "B.Cu") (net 4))
 (segment (start 155.851471 87.7) (end 155.951471 87.8) (width 0.3) (layer "F.Cu") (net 36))
 (segment (start 156.8 86.35) (end 156.367892 85.917892) (width 0.3) (layer "F.Cu") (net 36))
 (segment (start 154.8 87.7) (end 155.851471 87.7) (width 0.3) (layer "F.Cu") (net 36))
 (segment (start 156.367892 85.917892) (end 156.367892 77.082107) (width 0.3) (layer "F.Cu") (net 36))
 (segment (start 156.367892 77.082107) (end 151.19 71.904215) (width 0.3) (layer "F.Cu") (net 36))
 (segment (start 156.8 87.45) (end 156.8 86.35) (width 0.3) (layer "F.Cu") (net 36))
 (segment (start 156.45 87.8) (end 156.8 87.45) (width 0.3) (layer "F.Cu") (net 36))
 (segment (start 155.951471 87.8) (end 156.45 87.8) (width 0.3) (layer "F.Cu") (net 36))
 (segment (start 151.19 71.904215) (end 151.19 67.905) (width 0.3) (layer "F.Cu") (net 36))
 (segment (start 142.19 75.15) (end 142.19 85.99) (width 0.3) (layer "F.Cu") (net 7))
 (segment (start 142.4 86.2) (end 143.4 86.2) (width 0.3) (layer "F.Cu") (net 7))
 (segment (start 142.19 67.905) (end 142.19 75.15) (width 0.3) (layer "F.Cu") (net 7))
 (segment (start 142.19 85.99) (end 142.4 86.2) (width 0.3) (layer "F.Cu") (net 7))
 (via (at 142.19 75.15) (size 0.6) (drill 0.3) (layers "F.Cu" "B.Cu") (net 7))
 (segment (start 161.19 75.15) (end 161.19 67.905) (width 0.3) (layer "B.Cu") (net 7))
 (segment (start 142.19 75.15) (end 161.19 75.15) (width 0.3) (layer "B.Cu") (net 7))
 (segment (start 158.7 92) (end 158 92.7) (width 0.3) (layer "F.Cu") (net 33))
 (segment (start 158.7 76.35) (end 158.7 92) (width 0.3) (layer "F.Cu") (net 33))
 (segment (start 158 92.7) (end 154.8 92.7) (width 0.3) (layer "F.Cu") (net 33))
 (segment (start 156.14 67.905) (end 156.14 73.79) (width 0.3) (layer "F.Cu") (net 33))
 (segment (start 156.14 73.79) (end 158.7 76.35) (width 0.3) (layer "F.Cu") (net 33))
 (segment (start 141.16 76.76) (end 141.15 76.75) (width 0.3) (layer "F.Cu") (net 42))
 (segment (start 157.75 88.3) (end 157.75 84.25) (width 0.3) (layer "F.Cu") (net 42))
 (segment (start 155.85 90.2) (end 157.75 88.3) (width 0.3) (layer "F.Cu") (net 42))
 (segment (start 157.75 84.25) (end 157.75 77.05) (width 0.3) (layer "F.Cu") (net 42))
 (segment (start 157.75 77.05) (end 157.5 76.8) (width 0.3) (layer "F.Cu") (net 42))
 (segment (start 154.8 90.2) (end 155.85 90.2) (width 0.3) (layer "F.Cu") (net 42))
 (segment (start 141.15 76.75) (end 141.15 67.865) (width 0.3) (layer "F.Cu") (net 42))
 (segment (start 141.16 76.16) (end 141.16 76.76) (width 0.2) (layer "F.Cu") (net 42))
 (via (at 157.5 76.8) (size 0.6) (drill 0.3) (layers "F.Cu" "B.Cu") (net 42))
 (via (at 141.16 76.76) (size 0.6) (drill 0.3) (layers "F.Cu" "B.Cu") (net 42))
 (segment (start 141.2 76.8) (end 157.5 76.8) (width 0.3) (layer "B.Cu") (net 42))
 (segment (start 143.19 67.905) (end 143.19 77.56) (width 0.3) (layer "F.Cu") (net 11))
 (segment (start 143.19 77.56) (end 143.15 77.6) (width 0.2) (layer "F.Cu") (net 11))
 (segment (start 141.1 85.465686) (end 142.334314 86.7) (width 0.3) (layer "F.Cu") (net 11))
 (segment (start 142.334314 86.7) (end 143.4 86.7) (width 0.3) (layer "F.Cu") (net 11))
 (segment (start 141.1 77.65) (end 141.1 85.465686) (width 0.3) (layer "F.Cu") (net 11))
 (via (at 143.15 77.6) (size 0.6) (drill 0.3) (layers "F.Cu" "B.Cu") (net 11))
 (via (at 141.1 77.65) (size 0.6) (drill 0.3) (layers "F.Cu" "B.Cu") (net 11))
 (segment (start 141.15 77.6) (end 141.1 77.65) (width 0.2) (layer "B.Cu") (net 11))
 (segment (start 143.15 77.6) (end 141.15 77.6) (width 0.3) (layer "B.Cu") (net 11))
 (segment (start 134.875 89.2) (end 143.4 89.2) (width 0.3) (layer "F.Cu") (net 38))
 (segment (start 138.35 73.4) (end 134.875 76.875) (width 0.3) (layer "F.Cu") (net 38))
 (segment (start 149.19 73.24) (end 149.2 73.25) (width 0.2) (layer "F.Cu") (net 38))
 (segment (start 134.875 76.875) (end 134.875 89.2) (width 0.3) (layer "F.Cu") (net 38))
 (segment (start 149.19 67.905) (end 149.19 73.24) (width 0.3) (layer "F.Cu") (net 38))
 (via (at 138.35 73.4) (size 0.6) (drill 0.3) (layers "F.Cu" "B.Cu") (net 38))
 (via (at 149.2 73.25) (size 0.6) (drill 0.3) (layers "F.Cu" "B.Cu") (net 38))
 (segment (start 149.2 73.25) (end 138.5 73.25) (width 0.3) (layer "B.Cu") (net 38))
 (segment (start 138.5 73.25) (end 138.35 73.4) (width 0.2) (layer "B.Cu") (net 38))
 (segment (start 157.2 93.2) (end 157.49 93.49) (width 0.3) (layer "F.Cu") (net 32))
 (segment (start 154.8 93.2) (end 157.2 93.2) (width 0.3) (layer "F.Cu") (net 32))
 (segment (start 159.24 93.49) (end 159.24 67.905) (width 0.3) (layer "F.Cu") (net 32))
 (segment (start 157.49 93.49) (end 159.24 93.49) (width 0.3) (layer "F.Cu") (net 32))
 (segment (start 133.75 89.45) (end 134 89.7) (width 0.3) (layer "F.Cu") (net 37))
 (segment (start 133.75 77) (end 133.75 89.45) (width 0.3) (layer "F.Cu") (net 37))
 (segment (start 134 89.7) (end 143.4 89.7) (width 0.3) (layer "F.Cu") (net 37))
 (segment (start 138.15 72.6) (end 133.75 77) (width 0.3) (layer "F.Cu") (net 37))
 (segment (start 150.19 72.45) (end 150.19 67.905) (width 0.3) (layer "F.Cu") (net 37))
 (segment (start 138.15 72.5) (end 138.15 72.6) (width 0.2) (layer "F.Cu") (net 37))
 (via (at 138.15 72.5) (size 0.6) (drill 0.3) (layers "F.Cu" "B.Cu") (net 37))
 (via (at 150.19 72.45) (size 0.6) (drill 0.3) (layers "F.Cu" "B.Cu") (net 37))
 (segment (start 150.19 72.45) (end 138.2 72.45) (width 0.3) (layer "B.Cu") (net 37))
 (segment (start 138.2 72.45) (end 138.15 72.5) (width 0.2) (layer "B.Cu") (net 37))
 (segment (start 158.2 76.557106) (end 155.64 73.997106) (width 0.3) (layer "F.Cu") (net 34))
 (segment (start 158.2 91.4) (end 158.2 76.557106) (width 0.3) (layer "F.Cu") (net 34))
 (segment (start 155.19 73.476396) (end 155.19 67.905) (width 0.3) (layer "F.Cu") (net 34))
 (segment (start 155.64 73.926396) (end 155.19 73.476396) (width 0.3) (layer "F.Cu") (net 34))
 (segment (start 157.4 92.2) (end 158.2 91.4) (width 0.3) (layer "F.Cu") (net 34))
 (segment (start 155.64 73.997106) (end 155.64 73.926396) (width 0.3) (layer "F.Cu") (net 34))
 (segment (start 154.8 92.2) (end 157.4 92.2) (width 0.3) (layer "F.Cu") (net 34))
 (segment (start 139.19 74.21) (end 135.6 77.8) (width 0.3) (layer "F.Cu") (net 23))
 (segment (start 139.19 71.65) (end 139.19 74.21) (width 0.3) (layer "F.Cu") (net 23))
 (segment (start 135.6 77.8) (end 135.6 80.45) (width 0.3) (layer "F.Cu") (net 23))
 (via (at 139.19 71.65) (size 0.6) (drill 0.3) (layers "F.Cu" "B.Cu") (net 23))
 (segment (start 139.19 71.65) (end 139.19 67.905) (width 0.3) (layer "B.Cu") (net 23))
 (segment (start 156.2 87.2) (end 154.8 87.2) (width 0.3) (layer "F.Cu") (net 35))
 (segment (start 157.3 77.448529) (end 157.3 85.6) (width 0.3) (layer "F.Cu") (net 35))
 (segment (start 152.19 72.338529) (end 157.3 77.448529) (width 0.3) (layer "F.Cu") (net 35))
 (segment (start 152.19 67.905) (end 152.19 72.338529) (width 0.3) (layer "F.Cu") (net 35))
 (segment (start 157.3 85.6) (end 157.1 85.8) (width 0.3) (layer "F.Cu") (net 35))
 (via (at 156.2 87.2) (size 0.6) (drill 0.3) (layers "F.Cu" "B.Cu") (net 35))
 (via (at 157.1 85.8) (size 0.6) (drill 0.3) (layers "F.Cu" "B.Cu") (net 35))
 (segment (start 157.1 86.3) (end 156.2 87.2) (width 0.3) (layer "B.Cu") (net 35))
 (segment (start 157.1 85.8) (end 157.1 86.3) (width 0.3) (layer "B.Cu") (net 35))
 (segment (start 135.65 87.7) (end 137.3 87.7) (width 0.3) (layer "F.Cu") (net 71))
 (segment (start 135.65 82) (end 135.65 87.7) (width 0.3) (layer "F.Cu") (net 71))
 (segment (start 137.3 87.7) (end 143.4 87.7) (width 0.3) (layer "F.Cu") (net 71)))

